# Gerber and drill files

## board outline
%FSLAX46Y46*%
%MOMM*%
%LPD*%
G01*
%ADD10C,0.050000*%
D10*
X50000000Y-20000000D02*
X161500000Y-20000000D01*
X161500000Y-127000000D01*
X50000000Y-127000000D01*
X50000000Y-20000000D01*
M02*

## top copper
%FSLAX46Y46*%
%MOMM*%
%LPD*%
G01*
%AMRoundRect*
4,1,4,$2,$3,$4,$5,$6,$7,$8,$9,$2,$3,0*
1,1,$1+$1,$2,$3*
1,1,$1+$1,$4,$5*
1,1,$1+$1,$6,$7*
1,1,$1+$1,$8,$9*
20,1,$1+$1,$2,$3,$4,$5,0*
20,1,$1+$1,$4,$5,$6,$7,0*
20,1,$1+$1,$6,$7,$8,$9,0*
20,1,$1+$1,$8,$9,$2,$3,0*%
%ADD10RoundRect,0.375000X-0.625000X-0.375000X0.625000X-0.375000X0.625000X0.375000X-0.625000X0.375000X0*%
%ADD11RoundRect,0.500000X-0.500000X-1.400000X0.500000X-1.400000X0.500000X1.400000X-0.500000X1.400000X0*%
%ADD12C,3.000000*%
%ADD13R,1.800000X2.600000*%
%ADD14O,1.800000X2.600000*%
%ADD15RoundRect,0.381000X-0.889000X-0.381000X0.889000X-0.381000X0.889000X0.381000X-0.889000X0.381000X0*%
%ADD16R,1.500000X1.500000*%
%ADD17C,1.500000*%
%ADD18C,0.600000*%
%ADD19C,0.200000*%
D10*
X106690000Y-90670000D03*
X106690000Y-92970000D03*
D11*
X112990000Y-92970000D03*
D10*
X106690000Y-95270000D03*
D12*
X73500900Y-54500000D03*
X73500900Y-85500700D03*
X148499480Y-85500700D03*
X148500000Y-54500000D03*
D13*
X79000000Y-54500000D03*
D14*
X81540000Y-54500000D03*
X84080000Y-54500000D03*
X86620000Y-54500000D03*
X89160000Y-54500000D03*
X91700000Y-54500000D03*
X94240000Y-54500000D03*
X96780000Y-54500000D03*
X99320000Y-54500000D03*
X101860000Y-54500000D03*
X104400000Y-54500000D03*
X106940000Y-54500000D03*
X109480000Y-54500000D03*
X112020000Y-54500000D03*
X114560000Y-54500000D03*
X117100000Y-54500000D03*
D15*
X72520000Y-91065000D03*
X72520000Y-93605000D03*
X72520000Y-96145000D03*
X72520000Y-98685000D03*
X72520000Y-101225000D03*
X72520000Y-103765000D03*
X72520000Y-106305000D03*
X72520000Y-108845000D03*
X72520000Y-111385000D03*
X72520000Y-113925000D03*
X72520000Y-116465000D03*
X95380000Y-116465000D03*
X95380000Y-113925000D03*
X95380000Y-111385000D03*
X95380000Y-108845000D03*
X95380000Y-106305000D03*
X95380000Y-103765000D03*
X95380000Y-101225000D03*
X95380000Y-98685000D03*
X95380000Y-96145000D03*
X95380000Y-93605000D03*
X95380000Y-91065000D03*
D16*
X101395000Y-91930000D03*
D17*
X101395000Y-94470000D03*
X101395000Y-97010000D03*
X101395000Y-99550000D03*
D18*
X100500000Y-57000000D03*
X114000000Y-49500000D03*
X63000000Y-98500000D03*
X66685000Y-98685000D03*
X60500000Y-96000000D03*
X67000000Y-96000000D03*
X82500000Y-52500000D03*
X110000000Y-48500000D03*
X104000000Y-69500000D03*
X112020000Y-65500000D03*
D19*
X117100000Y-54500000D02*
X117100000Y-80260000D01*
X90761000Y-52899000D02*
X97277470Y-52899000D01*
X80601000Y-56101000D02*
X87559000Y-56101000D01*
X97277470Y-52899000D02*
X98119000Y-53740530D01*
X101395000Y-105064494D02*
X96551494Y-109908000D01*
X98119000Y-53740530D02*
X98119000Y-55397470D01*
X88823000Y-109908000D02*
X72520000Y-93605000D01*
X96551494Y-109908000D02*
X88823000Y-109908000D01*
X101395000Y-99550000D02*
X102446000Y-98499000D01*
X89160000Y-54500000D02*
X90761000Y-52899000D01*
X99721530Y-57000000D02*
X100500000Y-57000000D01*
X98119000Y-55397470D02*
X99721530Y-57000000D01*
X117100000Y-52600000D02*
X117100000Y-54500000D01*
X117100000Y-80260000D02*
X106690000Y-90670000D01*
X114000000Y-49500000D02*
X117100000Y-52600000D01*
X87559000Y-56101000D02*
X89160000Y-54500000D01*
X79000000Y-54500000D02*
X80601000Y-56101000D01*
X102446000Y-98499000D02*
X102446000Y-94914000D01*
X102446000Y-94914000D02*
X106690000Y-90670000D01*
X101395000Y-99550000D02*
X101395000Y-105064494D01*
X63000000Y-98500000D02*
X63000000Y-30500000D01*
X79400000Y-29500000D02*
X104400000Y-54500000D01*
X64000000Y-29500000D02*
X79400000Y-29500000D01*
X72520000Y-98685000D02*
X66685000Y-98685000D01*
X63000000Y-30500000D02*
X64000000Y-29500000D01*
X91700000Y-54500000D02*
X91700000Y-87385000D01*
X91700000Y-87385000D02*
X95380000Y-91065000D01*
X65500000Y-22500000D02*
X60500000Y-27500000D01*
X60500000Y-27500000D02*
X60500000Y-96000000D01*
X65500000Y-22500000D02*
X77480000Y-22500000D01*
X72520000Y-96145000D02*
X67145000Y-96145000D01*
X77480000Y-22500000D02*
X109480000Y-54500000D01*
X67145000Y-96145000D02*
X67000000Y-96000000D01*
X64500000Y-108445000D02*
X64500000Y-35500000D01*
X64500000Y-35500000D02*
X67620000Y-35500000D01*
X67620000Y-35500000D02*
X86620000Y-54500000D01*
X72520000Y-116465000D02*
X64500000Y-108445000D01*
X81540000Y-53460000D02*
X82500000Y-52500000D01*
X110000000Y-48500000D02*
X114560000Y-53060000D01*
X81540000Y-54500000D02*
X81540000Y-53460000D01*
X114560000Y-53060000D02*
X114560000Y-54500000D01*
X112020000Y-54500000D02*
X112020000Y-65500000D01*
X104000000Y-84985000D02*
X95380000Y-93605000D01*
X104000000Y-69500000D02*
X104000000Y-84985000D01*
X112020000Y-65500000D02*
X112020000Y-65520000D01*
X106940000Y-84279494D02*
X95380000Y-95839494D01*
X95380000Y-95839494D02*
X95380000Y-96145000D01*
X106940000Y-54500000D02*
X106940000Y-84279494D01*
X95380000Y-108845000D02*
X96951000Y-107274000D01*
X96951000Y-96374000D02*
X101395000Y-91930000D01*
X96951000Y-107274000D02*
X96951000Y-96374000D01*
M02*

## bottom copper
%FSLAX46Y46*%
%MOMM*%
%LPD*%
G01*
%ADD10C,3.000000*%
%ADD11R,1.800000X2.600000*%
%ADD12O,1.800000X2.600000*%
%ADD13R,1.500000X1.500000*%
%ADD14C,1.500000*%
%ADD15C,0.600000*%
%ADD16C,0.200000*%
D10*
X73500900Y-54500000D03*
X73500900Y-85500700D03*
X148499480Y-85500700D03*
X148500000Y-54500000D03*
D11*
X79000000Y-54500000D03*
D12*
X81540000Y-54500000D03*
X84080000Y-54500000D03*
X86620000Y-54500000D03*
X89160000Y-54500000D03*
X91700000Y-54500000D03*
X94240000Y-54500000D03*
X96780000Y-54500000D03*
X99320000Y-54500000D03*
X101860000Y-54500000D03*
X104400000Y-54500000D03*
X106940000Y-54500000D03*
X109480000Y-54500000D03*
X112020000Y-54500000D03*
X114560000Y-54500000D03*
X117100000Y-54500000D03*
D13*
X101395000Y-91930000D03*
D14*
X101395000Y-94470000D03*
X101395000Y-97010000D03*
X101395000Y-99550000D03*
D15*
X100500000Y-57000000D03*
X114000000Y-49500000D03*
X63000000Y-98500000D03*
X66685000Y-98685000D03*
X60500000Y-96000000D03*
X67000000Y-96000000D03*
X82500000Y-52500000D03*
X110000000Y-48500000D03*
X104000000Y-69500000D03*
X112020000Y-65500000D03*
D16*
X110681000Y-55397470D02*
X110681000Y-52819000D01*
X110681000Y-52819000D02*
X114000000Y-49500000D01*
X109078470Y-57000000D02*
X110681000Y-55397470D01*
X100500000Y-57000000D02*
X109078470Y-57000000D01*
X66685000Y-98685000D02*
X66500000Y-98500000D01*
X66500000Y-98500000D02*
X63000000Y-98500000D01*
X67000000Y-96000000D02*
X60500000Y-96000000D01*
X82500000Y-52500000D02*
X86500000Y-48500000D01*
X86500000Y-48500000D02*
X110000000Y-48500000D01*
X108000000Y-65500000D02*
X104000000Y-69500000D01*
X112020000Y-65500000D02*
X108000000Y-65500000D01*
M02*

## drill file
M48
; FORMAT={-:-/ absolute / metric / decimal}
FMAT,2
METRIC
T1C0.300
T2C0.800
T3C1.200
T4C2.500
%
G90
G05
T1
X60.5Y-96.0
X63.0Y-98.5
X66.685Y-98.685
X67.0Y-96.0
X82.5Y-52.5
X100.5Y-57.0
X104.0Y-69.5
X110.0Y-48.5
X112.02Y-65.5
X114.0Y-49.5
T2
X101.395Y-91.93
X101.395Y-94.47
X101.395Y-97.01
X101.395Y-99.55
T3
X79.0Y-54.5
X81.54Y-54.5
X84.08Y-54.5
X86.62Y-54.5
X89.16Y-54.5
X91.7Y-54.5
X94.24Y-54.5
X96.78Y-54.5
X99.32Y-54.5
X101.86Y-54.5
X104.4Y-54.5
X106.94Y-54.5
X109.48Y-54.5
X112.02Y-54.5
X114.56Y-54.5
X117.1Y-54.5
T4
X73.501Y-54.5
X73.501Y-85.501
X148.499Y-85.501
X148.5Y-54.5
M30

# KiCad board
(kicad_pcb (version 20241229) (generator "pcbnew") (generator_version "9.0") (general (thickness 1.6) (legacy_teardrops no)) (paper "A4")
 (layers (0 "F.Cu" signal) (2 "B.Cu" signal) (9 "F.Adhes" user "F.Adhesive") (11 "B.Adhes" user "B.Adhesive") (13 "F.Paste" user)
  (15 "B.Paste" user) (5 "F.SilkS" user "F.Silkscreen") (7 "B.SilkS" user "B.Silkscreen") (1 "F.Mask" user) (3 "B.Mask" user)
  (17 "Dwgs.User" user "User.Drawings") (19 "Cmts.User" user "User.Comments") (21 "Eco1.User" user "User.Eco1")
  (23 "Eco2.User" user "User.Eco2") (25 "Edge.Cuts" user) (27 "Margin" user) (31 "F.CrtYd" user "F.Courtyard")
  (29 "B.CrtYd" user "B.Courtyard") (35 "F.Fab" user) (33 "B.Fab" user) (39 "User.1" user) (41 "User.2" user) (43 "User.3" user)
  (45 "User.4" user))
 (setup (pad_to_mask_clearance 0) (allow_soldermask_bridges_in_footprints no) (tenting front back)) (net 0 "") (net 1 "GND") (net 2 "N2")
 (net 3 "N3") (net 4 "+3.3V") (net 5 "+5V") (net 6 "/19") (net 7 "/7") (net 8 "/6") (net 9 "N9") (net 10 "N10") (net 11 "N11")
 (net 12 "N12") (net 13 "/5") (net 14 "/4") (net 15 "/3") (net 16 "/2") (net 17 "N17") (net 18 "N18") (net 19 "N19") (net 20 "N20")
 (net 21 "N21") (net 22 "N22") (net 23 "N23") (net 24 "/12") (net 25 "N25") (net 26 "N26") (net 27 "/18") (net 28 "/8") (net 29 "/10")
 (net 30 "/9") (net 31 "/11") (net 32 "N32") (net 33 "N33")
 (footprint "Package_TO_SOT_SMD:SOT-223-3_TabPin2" (layer "F.Cu") (at 109.84 92.97)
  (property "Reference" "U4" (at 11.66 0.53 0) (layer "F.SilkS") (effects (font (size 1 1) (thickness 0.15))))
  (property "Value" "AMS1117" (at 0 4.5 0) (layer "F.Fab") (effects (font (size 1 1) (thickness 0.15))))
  (pad "1" smd roundrect (at -3.15 -2.3) (size 2 1.5) (layers "F.Cu" "F.Mask" "F.Paste") (roundrect_rratio 0.25) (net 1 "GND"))
  (pad "2" smd roundrect (at -3.15 0) (size 2 1.5) (layers "F.Cu" "F.Mask" "F.Paste") (roundrect_rratio 0.25) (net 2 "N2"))
  (pad "2" smd roundrect (at 3.15 0) (size 2 3.8) (layers "F.Cu" "F.Mask" "F.Paste") (roundrect_rratio 0.25) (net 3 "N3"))
  (pad "3" smd roundrect (at -3.15 2.3) (size 2 1.5) (layers "F.Cu" "F.Mask" "F.Paste") (roundrect_rratio 0.25) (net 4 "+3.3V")))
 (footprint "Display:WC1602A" (layer "F.Cu") (at 79 54.5)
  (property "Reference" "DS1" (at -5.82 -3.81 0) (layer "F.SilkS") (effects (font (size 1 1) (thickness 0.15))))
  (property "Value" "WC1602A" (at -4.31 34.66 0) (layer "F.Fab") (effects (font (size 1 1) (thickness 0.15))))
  (pad "" thru_hole circle (at -5.4991 0) (size 3 3) (drill 2.5) (layers "*.Cu" "*.Mask") (remove_unused_layers no))
  (pad "" thru_hole circle (at -5.4991 31.0007) (size 3 3) (drill 2.5) (layers "*.Cu" "*.Mask") (remove_unused_layers no))
  (pad "" thru_hole circle (at 69.49948 31.0007) (size 3 3) (drill 2.5) (layers "*.Cu" "*.Mask") (remove_unused_layers no))
  (pad "" thru_hole circle (at 69.5 0) (size 3 3) (drill 2.5) (layers "*.Cu" "*.Mask") (remove_unused_layers no))
  (pad "1" thru_hole rect (at 0 0) (size 1.8 2.6) (drill 1.2) (layers "*.Cu" "*.Mask") (remove_unused_layers no) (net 1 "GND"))
  (pad "2" thru_hole oval (at 2.54 0) (size 1.8 2.6) (drill 1.2) (layers "*.Cu" "*.Mask") (remove_unused_layers no) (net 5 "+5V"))
  (pad "3" thru_hole oval (at 5.08 0) (size 1.8 2.6) (drill 1.2) (layers "*.Cu" "*.Mask") (remove_unused_layers no) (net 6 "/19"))
  (pad "4" thru_hole oval (at 7.62 0) (size 1.8 2.6) (drill 1.2) (layers "*.Cu" "*.Mask") (remove_unused_layers no) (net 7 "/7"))
  (pad "5" thru_hole oval (at 10.16 0) (size 1.8 2.6) (drill 1.2) (layers "*.Cu" "*.Mask") (remove_unused_layers no) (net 1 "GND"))
  (pad "6" thru_hole oval (at 12.7 0) (size 1.8 2.6) (drill 1.2) (layers "*.Cu" "*.Mask") (remove_unused_layers no) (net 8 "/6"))
  (pad "7" thru_hole oval (at 15.24 0) (size 1.8 2.6) (drill 1.2) (layers "*.Cu" "*.Mask") (remove_unused_layers no) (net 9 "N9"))
  (pad "8" thru_hole oval (at 17.78 0) (size 1.8 2.6) (drill 1.2) (layers "*.Cu" "*.Mask") (remove_unused_layers no) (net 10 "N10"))
  (pad "9" thru_hole oval (at 20.32 0) (size 1.8 2.6) (drill 1.2) (layers "*.Cu" "*.Mask") (remove_unused_layers no) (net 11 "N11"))
  (pad "10" thru_hole oval (at 22.86 0) (size 1.8 2.6) (drill 1.2) (layers "*.Cu" "*.Mask") (remove_unused_layers no) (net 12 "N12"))
  (pad "11" thru_hole oval (at 25.4 0) (size 1.8 2.6) (drill 1.2) (layers "*.Cu" "*.Mask") (remove_unused_layers no) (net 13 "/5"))
  (pad "12" thru_hole oval (at 27.94 0) (size 1.8 2.6) (drill 1.2) (layers "*.Cu" "*.Mask") (remove_unused_layers no) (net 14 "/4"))
  (pad "13" thru_hole oval (at 30.48 0) (size 1.8 2.6) (drill 1.2) (layers "*.Cu" "*.Mask") (remove_unused_layers no) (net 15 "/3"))
  (pad "14" thru_hole oval (at 33.02 0) (size 1.8 2.6) (drill 1.2) (layers "*.Cu" "*.Mask") (remove_unused_layers no) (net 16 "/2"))
  (pad "15" thru_hole oval (at 35.56 0) (size 1.8 2.6) (drill 1.2) (layers "*.Cu" "*.Mask") (remove_unused_layers no) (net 5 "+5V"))
  (pad "16" thru_hole oval (at 38.1 0) (size 1.8 2.6) (drill 1.2) (layers "*.Cu" "*.Mask") (remove_unused_layers no) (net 1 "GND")))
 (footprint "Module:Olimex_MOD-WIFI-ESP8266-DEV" (layer "F.Cu") (at 83.95 103.765)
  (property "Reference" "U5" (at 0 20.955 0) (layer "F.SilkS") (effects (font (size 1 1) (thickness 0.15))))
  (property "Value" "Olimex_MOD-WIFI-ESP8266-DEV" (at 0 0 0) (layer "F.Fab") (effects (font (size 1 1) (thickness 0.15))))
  (pad "1" smd roundrect (at -11.43 -12.7) (size 2.54 1.524) (layers "F.Cu" "F.Mask" "F.Paste") (roundrect_rratio 0.25) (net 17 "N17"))
  (pad "2" smd roundrect (at -11.43 -10.16) (size 2.54 1.524) (layers "F.Cu" "F.Mask" "F.Paste") (roundrect_rratio 0.25) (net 1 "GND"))
  (pad "3" smd roundrect (at -11.43 -7.62) (size 2.54 1.524) (layers "F.Cu" "F.Mask" "F.Paste") (roundrect_rratio 0.25) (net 15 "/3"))
  (pad "4" smd roundrect (at -11.43 -5.08) (size 2.54 1.524) (layers "F.Cu" "F.Mask" "F.Paste") (roundrect_rratio 0.25) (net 13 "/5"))
  (pad "5" smd roundrect (at -11.43 -2.54) (size 2.54 1.524) (layers "F.Cu" "F.Mask" "F.Paste") (roundrect_rratio 0.25) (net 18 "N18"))
  (pad "6" smd roundrect (at -11.43 0) (size 2.54 1.524) (layers "F.Cu" "F.Mask" "F.Paste") (roundrect_rratio 0.25) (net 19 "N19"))
  (pad "7" smd roundrect (at -11.43 2.54) (size 2.54 1.524) (layers "F.Cu" "F.Mask" "F.Paste") (roundrect_rratio 0.25) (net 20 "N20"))
  (pad "8" smd roundrect (at -11.43 5.08) (size 2.54 1.524) (layers "F.Cu" "F.Mask" "F.Paste") (roundrect_rratio 0.25) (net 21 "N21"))
  (pad "9" smd roundrect (at -11.43 7.62) (size 2.54 1.524) (layers "F.Cu" "F.Mask" "F.Paste") (roundrect_rratio 0.25) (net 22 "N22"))
  (pad "10" smd roundrect (at -11.43 10.16) (size 2.54 1.524) (layers "F.Cu" "F.Mask" "F.Paste") (roundrect_rratio 0.25) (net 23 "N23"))
  (pad "11" smd roundrect (at -11.43 12.7) (size 2.54 1.524) (layers "F.Cu" "F.Mask" "F.Paste") (roundrect_rratio 0.25) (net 7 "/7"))
  (pad "12" smd roundrect (at 11.43 12.7) (size 2.54 1.524) (layers "F.Cu" "F.Mask" "F.Paste") (roundrect_rratio 0.25) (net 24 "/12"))
  (pad "13" smd roundrect (at 11.43 10.16) (size 2.54 1.524) (layers "F.Cu" "F.Mask" "F.Paste") (roundrect_rratio 0.25) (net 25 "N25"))
  (pad "14" smd roundrect (at 11.43 7.62) (size 2.54 1.524) (layers "F.Cu" "F.Mask" "F.Paste") (roundrect_rratio 0.25) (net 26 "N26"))
  (pad "15" smd roundrect (at 11.43 5.08) (size 2.54 1.524) (layers "F.Cu" "F.Mask" "F.Paste") (roundrect_rratio 0.25) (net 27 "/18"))
  (pad "16" smd roundrect (at 11.43 2.54) (size 2.54 1.524) (layers "F.Cu" "F.Mask" "F.Paste") (roundrect_rratio 0.25) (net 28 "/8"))
  (pad "17" smd roundrect (at 11.43 0) (size 2.54 1.524) (layers "F.Cu" "F.Mask" "F.Paste") (roundrect_rratio 0.25) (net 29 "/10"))
  (pad "18" smd roundrect (at 11.43 -2.54) (size 2.54 1.524) (layers "F.Cu" "F.Mask" "F.Paste") (roundrect_rratio 0.25) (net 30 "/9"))
  (pad "19" smd roundrect (at 11.43 -5.08) (size 2.54 1.524) (layers "F.Cu" "F.Mask" "F.Paste") (roundrect_rratio 0.25) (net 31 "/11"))
  (pad "20" smd roundrect (at 11.43 -7.62) (size 2.54 1.524) (layers "F.Cu" "F.Mask" "F.Paste") (roundrect_rratio 0.25) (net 14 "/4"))
  (pad "21" smd roundrect (at 11.43 -10.16) (size 2.54 1.524) (layers "F.Cu" "F.Mask" "F.Paste") (roundrect_rratio 0.25) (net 16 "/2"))
  (pad "22" smd roundrect (at 11.43 -12.7) (size 2.54 1.524) (layers "F.Cu" "F.Mask" "F.Paste") (roundrect_rratio 0.25) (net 8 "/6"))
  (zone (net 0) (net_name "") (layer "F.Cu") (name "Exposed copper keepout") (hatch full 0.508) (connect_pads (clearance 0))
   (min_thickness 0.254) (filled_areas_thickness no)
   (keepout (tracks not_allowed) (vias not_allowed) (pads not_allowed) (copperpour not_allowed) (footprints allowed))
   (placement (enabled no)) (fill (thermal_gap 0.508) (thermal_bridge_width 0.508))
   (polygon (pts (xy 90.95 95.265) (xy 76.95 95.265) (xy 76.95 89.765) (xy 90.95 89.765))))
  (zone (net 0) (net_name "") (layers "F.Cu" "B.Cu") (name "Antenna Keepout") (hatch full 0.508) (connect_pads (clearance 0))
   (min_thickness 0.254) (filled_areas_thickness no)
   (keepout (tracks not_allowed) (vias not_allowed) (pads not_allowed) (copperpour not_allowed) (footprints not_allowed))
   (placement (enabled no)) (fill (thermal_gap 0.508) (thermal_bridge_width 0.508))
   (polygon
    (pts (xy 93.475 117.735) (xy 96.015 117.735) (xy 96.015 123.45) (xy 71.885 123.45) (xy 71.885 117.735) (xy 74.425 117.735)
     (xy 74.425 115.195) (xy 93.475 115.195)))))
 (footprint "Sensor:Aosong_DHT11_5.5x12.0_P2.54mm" (layer "F.Cu") (at 101.395 91.93)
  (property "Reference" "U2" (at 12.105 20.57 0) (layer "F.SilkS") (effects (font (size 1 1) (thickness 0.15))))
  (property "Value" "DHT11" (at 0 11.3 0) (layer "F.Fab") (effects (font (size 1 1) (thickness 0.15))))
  (pad "1" thru_hole rect (at 0 0) (size 1.5 1.5) (drill 0.8) (layers "*.Cu" "*.Mask") (remove_unused_layers no) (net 27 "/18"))
  (pad "2" thru_hole circle (at 0 2.54) (size 1.5 1.5) (drill 0.8) (layers "*.Cu" "*.Mask") (remove_unused_layers no) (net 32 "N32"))
  (pad "3" thru_hole circle (at 0 5.08) (size 1.5 1.5) (drill 0.8) (layers "*.Cu" "*.Mask") (remove_unused_layers no) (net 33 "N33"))
  (pad "4" thru_hole circle (at 0 7.62) (size 1.5 1.5) (drill 0.8) (layers "*.Cu" "*.Mask") (remove_unused_layers no) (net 1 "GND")))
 (gr_rect (start 50 20) (end 161.5 127) (stroke (width 0.05) (type default)) (fill no) (layer "Edge.Cuts"))
 (segment (start 117.1 54.5) (end 117.1 80.26) (width 0.2) (layer "F.Cu") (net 1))
 (segment (start 90.761 52.899) (end 97.27747 52.899) (width 0.2) (layer "F.Cu") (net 1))
 (segment (start 80.601 56.101) (end 87.559 56.101) (width 0.2) (layer "F.Cu") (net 1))
 (segment (start 97.27747 52.899) (end 98.119 53.74053) (width 0.2) (layer "F.Cu") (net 1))
 (segment (start 101.395 105.064494) (end 96.551494 109.908) (width 0.2) (layer "F.Cu") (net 1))
 (segment (start 98.119 53.74053) (end 98.119 55.39747) (width 0.2) (layer "F.Cu") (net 1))
 (segment (start 88.823 109.908) (end 72.52 93.605) (width 0.2) (layer "F.Cu") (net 1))
 (segment (start 96.551494 109.908) (end 88.823 109.908) (width 0.2) (layer "F.Cu") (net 1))
 (segment (start 101.395 99.55) (end 102.446 98.499) (width 0.2) (layer "F.Cu") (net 1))
 (segment (start 89.16 54.5) (end 90.761 52.899) (width 0.2) (layer "F.Cu") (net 1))
 (segment (start 99.72153 57) (end 100.5 57) (width 0.2) (layer "F.Cu") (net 1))
 (segment (start 98.119 55.39747) (end 99.72153 57) (width 0.2) (layer "F.Cu") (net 1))
 (segment (start 117.1 52.6) (end 117.1 54.5) (width 0.2) (layer "F.Cu") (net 1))
 (segment (start 117.1 80.26) (end 106.69 90.67) (width 0.2) (layer "F.Cu") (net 1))
 (segment (start 114 49.5) (end 117.1 52.6) (width 0.2) (layer "F.Cu") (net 1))
 (segment (start 87.559 56.101) (end 89.16 54.5) (width 0.2) (layer "F.Cu") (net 1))
 (segment (start 79 54.5) (end 80.601 56.101) (width 0.2) (layer "F.Cu") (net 1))
 (segment (start 102.446 98.499) (end 102.446 94.914) (width 0.2) (layer "F.Cu") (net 1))
 (segment (start 102.446 94.914) (end 106.69 90.67) (width 0.2) (layer "F.Cu") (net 1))
 (segment (start 101.395 99.55) (end 101.395 105.064494) (width 0.2) (layer "F.Cu") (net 1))
 (via (at 100.5 57) (size 0.6) (drill 0.3) (layers "F.Cu" "B.Cu") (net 1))
 (via (at 114 49.5) (size 0.6) (drill 0.3) (layers "F.Cu" "B.Cu") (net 1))
 (segment (start 110.681 55.39747) (end 110.681 52.819) (width 0.2) (layer "B.Cu") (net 1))
 (segment (start 110.681 52.819) (end 114 49.5) (width 0.2) (layer "B.Cu") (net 1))
 (segment (start 109.07847 57) (end 110.681 55.39747) (width 0.2) (layer "B.Cu") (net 1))
 (segment (start 100.5 57) (end 109.07847 57) (width 0.2) (layer "B.Cu") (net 1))
 (segment (start 63 98.5) (end 63 30.5) (width 0.2) (layer "F.Cu") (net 13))
 (segment (start 79.4 29.5) (end 104.4 54.5) (width 0.2) (layer "F.Cu") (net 13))
 (segment (start 64 29.5) (end 79.4 29.5) (width 0.2) (layer "F.Cu") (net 13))
 (segment (start 72.52 98.685) (end 66.685 98.685) (width 0.2) (layer "F.Cu") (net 13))
 (segment (start 63 30.5) (end 64 29.5) (width 0.2) (layer "F.Cu") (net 13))
 (via (at 63 98.5) (size 0.6) (drill 0.3) (layers "F.Cu" "B.Cu") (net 13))
 (via (at 66.685 98.685) (size 0.6) (drill 0.3) (layers "F.Cu" "B.Cu") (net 13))
 (segment (start 66.685 98.685) (end 66.5 98.5) (width 0.2) (layer "B.Cu") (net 13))
 (segment (start 66.5 98.5) (end 63 98.5) (width 0.2) (layer "B.Cu") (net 13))
 (segment (start 91.7 54.5) (end 91.7 87.385) (width 0.2) (layer "F.Cu") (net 8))
 (segment (start 91.7 87.385) (end 95.38 91.065) (width 0.2) (layer "F.Cu") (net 8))
 (segment (start 65.5 22.5) (end 60.5 27.5) (width 0.2) (layer "F.Cu") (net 15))
 (segment (start 60.5 27.5) (end 60.5 96) (width 0.2) (layer "F.Cu") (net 15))
 (segment (start 65.5 22.5) (end 77.48 22.5) (width 0.2) (layer "F.Cu") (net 15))
 (segment (start 72.52 96.145) (end 67.145 96.145) (width 0.2) (layer "F.Cu") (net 15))
 (segment (start 77.48 22.5) (end 109.48 54.5) (width 0.2) (layer "F.Cu") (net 15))
 (segment (start 67.145 96.145) (end 67 96) (width 0.2) (layer "F.Cu") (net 15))
 (via (at 60.5 96) (size 0.6) (drill 0.3) (layers "F.Cu" "B.Cu") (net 15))
 (via (at 67 96) (size 0.6) (drill 0.3) (layers "F.Cu" "B.Cu") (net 15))
 (segment (start 67 96) (end 60.5 96) (width 0.2) (layer "B.Cu") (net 15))
 (segment (start 64.5 108.445) (end 64.5 35.5) (width 0.2) (layer "F.Cu") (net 7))
 (segment (start 64.5 35.5) (end 67.62 35.5) (width 0.2) (layer "F.Cu") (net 7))
 (segment (start 67.62 35.5) (end 86.62 54.5) (width 0.2) (layer "F.Cu") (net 7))
 (segment (start 72.52 116.465) (end 64.5 108.445) (width 0.2) (layer "F.Cu") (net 7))
 (segment (start 81.54 53.46) (end 82.5 52.5) (width 0.2) (layer "F.Cu") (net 5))
 (segment (start 110 48.5) (end 114.56 53.06) (width 0.2) (layer "F.Cu") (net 5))
 (segment (start 81.54 54.5) (end 81.54 53.46) (width 0.2) (layer "F.Cu") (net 5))
 (segment (start 114.56 53.06) (end 114.56 54.5) (width 0.2) (layer "F.Cu") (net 5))
 (via (at 82.5 52.5) (size 0.6) (drill 0.3) (layers "F.Cu" "B.Cu") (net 5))
 (via (at 110 48.5) (size 0.6) (drill 0.3) (layers "F.Cu" "B.Cu") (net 5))
 (segment (start 82.5 52.5) (end 86.5 48.5) (width 0.2) (layer "B.Cu") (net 5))
 (segment (start 86.5 48.5) (end 110 48.5) (width 0.2) (layer "B.Cu") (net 5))
 (segment (start 112.02 54.5) (end 112.02 65.5) (width 0.2) (layer "F.Cu") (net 16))
 (segment (start 104 84.985) (end 95.38 93.605) (width 0.2) (layer "F.Cu") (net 16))
 (segment (start 104 69.5) (end 104 84.985) (width 0.2) (layer "F.Cu") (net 16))
 (segment (start 112.02 65.5) (end 112.02 65.52) (width 0.2) (layer "F.Cu") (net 16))
 (via (at 104 69.5) (size 0.6) (drill 0.3) (layers "F.Cu" "B.Cu") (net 16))
 (via (at 112.02 65.5) (size 0.6) (drill 0.3) (layers "F.Cu" "B.Cu") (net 16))
 (segment (start 108 65.5) (end 104 69.5) (width 0.2) (layer "B.Cu") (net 16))
 (segment (start 112.02 65.5) (end 108 65.5) (width 0.2) (layer "B.Cu") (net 16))
 (segment (start 106.94 84.279494) (end 95.38 95.839494) (width 0.2) (layer "F.Cu") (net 14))
 (segment (start 95.38 95.839494) (end 95.38 96.145) (width 0.2) (layer "F.Cu") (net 14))
 (segment (start 106.94 54.5) (end 106.94 84.279494) (width 0.2) (layer "F.Cu") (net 14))
 (segment (start 95.38 108.845) (end 96.951 107.274) (width 0.2) (layer "F.Cu") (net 27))
 (segment (start 96.951 96.374) (end 101.395 91.93) (width 0.2) (layer "F.Cu") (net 27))
 (segment (start 96.951 107.274) (end 96.951 96.374) (width 0.2) (layer "F.Cu") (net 27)))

